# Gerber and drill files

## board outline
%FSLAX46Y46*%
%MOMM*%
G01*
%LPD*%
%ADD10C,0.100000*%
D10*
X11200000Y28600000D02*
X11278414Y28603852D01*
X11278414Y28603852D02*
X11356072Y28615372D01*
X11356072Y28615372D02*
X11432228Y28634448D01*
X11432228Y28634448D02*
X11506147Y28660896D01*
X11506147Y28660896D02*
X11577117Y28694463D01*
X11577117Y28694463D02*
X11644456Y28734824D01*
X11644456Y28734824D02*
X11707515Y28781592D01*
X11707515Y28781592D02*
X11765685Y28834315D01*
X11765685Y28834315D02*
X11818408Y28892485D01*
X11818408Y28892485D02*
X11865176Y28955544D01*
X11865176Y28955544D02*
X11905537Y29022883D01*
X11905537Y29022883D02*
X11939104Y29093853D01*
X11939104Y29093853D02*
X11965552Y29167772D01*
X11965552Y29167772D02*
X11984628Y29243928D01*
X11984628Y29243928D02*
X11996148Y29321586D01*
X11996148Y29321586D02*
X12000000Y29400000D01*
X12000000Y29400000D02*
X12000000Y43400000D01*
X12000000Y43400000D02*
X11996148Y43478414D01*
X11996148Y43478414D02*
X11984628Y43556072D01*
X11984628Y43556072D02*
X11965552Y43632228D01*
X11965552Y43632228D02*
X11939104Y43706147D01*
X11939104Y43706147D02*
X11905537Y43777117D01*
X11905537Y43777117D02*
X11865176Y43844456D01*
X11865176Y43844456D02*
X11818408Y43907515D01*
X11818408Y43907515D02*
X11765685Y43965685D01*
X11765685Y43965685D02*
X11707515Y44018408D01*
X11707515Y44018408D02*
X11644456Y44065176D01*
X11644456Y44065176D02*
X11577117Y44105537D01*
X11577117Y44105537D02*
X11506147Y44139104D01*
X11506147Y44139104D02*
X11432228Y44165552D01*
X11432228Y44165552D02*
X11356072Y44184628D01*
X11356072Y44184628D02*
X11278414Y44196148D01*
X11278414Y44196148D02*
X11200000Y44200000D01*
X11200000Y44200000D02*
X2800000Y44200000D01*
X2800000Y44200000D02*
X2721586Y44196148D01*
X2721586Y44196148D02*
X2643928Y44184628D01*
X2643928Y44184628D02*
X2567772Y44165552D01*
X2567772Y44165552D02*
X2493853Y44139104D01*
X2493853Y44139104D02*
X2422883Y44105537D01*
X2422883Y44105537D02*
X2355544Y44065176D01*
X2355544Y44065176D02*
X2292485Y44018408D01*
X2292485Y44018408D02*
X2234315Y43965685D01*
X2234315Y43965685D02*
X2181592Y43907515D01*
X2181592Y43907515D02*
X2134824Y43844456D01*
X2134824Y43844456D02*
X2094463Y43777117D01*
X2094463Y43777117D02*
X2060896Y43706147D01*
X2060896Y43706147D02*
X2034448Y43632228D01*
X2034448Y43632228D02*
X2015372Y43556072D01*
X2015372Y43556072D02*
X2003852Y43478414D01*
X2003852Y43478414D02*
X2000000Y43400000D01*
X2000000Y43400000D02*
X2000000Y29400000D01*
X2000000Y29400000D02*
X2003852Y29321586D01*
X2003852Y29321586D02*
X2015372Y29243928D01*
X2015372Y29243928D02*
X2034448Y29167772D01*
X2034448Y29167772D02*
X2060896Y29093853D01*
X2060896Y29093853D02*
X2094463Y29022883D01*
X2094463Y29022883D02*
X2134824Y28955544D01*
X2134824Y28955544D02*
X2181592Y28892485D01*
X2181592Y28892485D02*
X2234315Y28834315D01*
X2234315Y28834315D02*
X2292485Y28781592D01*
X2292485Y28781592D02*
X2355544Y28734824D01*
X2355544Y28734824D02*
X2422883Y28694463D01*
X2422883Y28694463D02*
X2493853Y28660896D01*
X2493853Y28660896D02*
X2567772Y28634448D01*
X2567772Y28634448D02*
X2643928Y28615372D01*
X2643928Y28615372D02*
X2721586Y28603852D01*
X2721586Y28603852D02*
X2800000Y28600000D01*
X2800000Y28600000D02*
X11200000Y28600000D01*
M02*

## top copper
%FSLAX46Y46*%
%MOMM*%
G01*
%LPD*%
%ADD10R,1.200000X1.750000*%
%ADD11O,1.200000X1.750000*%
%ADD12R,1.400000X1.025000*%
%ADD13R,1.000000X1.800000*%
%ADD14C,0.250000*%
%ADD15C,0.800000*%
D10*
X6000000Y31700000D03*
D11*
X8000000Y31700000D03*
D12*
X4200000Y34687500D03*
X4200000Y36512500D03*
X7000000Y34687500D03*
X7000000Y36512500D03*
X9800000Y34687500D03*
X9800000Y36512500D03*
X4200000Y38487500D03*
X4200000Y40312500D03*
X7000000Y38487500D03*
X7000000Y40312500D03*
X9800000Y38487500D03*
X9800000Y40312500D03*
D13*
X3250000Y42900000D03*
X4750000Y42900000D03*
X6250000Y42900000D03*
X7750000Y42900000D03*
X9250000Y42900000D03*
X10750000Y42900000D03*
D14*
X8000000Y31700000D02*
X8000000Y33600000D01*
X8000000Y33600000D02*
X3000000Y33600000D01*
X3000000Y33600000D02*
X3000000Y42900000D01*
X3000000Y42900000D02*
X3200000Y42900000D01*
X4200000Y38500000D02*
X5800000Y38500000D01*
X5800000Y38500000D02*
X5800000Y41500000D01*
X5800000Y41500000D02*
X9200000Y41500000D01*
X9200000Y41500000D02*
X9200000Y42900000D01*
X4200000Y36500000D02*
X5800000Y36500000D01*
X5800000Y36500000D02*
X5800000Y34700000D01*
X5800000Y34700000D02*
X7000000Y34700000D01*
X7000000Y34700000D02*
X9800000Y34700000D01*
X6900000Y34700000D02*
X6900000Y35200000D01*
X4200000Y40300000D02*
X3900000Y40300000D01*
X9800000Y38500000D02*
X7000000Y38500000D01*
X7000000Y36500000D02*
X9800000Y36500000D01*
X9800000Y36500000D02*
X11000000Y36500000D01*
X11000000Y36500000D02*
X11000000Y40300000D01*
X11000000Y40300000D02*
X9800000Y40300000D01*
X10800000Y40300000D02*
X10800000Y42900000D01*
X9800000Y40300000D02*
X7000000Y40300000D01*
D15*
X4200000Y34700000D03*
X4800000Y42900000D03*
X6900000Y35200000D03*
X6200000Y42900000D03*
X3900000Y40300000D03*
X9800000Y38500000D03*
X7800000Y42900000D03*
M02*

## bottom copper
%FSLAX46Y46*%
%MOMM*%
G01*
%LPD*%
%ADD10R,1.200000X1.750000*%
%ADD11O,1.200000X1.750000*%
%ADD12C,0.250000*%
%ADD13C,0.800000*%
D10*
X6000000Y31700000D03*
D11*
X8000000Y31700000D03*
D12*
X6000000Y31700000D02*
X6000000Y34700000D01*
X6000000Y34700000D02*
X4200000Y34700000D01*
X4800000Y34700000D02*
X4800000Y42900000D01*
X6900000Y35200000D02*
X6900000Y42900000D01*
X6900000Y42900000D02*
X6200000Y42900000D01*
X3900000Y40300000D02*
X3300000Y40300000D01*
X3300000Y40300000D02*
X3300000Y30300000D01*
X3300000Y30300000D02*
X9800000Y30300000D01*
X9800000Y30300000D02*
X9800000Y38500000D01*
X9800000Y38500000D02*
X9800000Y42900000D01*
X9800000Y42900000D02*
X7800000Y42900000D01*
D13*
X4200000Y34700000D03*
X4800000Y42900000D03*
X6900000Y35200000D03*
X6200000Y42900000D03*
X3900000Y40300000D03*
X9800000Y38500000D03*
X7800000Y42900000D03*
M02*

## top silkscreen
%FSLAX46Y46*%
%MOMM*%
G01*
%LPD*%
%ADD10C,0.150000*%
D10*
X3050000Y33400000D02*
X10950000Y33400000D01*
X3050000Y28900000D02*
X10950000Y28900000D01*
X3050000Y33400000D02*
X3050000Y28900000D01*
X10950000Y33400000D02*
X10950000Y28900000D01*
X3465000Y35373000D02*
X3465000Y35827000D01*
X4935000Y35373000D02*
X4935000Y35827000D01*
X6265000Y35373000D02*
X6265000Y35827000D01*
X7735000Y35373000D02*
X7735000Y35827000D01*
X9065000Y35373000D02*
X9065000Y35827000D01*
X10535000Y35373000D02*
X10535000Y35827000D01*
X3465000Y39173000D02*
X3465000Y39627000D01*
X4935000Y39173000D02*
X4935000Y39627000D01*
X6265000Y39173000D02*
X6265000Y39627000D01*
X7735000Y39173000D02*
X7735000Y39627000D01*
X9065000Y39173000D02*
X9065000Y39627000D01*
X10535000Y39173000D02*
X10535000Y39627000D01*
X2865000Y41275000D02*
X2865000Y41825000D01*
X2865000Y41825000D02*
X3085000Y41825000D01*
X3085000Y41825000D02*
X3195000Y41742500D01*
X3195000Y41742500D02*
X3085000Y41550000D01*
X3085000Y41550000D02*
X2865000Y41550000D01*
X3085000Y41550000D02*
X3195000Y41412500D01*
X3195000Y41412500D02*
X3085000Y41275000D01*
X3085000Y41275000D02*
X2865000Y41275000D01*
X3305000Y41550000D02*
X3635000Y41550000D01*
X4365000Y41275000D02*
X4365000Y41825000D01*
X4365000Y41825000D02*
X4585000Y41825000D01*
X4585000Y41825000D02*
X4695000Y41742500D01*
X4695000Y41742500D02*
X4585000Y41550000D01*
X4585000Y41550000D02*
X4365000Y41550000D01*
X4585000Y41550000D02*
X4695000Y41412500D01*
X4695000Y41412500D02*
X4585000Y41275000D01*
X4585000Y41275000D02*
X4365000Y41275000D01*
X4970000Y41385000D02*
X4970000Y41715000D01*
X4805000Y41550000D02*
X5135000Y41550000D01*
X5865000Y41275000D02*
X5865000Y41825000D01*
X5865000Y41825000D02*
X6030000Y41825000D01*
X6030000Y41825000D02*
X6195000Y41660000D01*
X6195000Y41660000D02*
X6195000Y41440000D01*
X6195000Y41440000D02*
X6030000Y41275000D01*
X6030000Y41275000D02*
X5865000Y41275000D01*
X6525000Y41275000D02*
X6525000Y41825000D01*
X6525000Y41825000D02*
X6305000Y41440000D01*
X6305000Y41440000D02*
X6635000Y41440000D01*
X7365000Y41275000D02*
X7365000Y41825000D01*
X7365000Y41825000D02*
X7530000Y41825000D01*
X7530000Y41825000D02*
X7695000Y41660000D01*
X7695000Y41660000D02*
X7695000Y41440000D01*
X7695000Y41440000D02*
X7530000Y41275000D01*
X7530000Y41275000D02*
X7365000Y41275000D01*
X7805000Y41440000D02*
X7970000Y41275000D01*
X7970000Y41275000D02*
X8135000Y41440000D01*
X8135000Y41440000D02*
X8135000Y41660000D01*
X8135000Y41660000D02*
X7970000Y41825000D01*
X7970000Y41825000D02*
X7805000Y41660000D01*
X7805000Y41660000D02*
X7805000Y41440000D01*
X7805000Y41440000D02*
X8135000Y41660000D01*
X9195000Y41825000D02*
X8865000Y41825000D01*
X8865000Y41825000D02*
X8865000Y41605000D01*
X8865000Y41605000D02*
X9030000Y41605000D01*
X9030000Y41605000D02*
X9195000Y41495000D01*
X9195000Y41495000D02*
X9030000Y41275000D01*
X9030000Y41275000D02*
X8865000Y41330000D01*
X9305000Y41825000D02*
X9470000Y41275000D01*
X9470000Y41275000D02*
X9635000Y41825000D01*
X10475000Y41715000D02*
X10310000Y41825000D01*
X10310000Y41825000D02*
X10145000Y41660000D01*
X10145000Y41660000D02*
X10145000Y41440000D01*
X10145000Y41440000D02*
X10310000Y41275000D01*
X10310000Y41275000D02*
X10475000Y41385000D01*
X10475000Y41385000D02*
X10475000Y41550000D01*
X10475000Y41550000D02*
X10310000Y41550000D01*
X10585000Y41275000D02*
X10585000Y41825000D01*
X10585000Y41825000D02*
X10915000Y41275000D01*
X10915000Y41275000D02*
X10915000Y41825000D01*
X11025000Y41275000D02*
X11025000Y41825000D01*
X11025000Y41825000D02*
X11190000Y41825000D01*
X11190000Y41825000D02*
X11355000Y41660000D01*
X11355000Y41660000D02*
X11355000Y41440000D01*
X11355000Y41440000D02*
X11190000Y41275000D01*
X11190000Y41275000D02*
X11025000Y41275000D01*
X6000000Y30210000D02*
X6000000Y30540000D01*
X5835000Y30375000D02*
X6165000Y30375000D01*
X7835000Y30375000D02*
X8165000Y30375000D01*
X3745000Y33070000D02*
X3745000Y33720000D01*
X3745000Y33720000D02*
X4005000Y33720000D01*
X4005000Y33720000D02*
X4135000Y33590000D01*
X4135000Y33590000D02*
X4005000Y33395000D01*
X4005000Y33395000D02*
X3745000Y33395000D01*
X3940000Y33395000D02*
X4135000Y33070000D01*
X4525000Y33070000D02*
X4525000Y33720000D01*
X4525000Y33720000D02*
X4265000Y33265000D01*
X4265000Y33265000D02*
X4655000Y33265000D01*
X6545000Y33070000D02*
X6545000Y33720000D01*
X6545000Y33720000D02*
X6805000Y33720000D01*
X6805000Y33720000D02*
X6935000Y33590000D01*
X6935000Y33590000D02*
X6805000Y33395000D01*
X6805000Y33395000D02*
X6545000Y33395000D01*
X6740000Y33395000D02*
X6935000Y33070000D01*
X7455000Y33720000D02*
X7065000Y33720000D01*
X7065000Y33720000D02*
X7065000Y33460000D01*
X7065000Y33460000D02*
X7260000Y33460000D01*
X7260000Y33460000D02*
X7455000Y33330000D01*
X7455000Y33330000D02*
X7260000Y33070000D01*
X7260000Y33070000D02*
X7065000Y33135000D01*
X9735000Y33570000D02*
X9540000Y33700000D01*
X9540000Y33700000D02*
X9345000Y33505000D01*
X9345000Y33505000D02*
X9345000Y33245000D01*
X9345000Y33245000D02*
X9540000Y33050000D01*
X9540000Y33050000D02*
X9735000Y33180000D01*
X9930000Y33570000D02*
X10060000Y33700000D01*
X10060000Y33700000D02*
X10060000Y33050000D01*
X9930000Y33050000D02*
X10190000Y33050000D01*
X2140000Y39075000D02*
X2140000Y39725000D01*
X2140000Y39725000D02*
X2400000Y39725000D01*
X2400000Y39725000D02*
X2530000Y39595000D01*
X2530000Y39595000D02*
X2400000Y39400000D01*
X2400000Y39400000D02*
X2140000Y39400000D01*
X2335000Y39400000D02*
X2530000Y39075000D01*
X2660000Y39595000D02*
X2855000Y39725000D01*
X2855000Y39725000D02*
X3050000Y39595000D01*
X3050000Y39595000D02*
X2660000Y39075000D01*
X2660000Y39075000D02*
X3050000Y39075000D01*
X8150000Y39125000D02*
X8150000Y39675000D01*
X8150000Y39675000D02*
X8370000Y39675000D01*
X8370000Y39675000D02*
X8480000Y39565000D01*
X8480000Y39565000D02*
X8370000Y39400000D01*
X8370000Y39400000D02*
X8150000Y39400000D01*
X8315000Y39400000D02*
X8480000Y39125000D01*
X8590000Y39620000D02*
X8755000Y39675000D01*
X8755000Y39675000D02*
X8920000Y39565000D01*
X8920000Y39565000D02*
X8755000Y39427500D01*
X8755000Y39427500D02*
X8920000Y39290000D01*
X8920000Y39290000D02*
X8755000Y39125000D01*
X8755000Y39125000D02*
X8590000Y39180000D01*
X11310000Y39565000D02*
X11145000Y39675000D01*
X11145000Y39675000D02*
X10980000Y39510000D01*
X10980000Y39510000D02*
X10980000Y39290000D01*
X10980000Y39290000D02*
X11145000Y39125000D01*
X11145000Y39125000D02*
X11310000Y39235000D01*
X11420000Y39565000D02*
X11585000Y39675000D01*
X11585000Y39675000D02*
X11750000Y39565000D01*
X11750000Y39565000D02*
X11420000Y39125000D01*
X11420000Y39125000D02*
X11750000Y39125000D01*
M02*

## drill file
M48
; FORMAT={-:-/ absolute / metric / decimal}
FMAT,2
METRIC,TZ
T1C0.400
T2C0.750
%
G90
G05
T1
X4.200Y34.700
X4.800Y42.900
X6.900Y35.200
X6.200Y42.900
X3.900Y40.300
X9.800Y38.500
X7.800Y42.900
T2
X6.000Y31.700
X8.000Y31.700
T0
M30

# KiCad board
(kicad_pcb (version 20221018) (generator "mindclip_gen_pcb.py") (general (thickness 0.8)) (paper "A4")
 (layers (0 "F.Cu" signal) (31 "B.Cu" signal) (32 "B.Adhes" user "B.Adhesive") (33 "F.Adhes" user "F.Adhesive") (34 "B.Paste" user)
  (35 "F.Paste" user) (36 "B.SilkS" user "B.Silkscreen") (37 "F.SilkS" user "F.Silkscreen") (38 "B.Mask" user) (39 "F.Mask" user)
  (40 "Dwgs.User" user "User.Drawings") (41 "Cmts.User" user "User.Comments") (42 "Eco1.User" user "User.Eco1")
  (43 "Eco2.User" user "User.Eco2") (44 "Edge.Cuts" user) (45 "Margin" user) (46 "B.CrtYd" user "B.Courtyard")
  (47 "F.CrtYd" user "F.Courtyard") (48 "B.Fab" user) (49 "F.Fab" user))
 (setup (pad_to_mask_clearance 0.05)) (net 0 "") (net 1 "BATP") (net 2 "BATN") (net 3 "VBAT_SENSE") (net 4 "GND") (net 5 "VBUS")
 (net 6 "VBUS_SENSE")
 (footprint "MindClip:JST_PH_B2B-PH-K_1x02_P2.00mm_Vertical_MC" (layer "F.Cu") (at 37 88.3)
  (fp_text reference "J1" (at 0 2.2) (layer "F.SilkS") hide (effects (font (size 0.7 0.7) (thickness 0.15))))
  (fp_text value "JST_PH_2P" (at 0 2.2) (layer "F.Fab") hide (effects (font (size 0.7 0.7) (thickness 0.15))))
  (fp_line (start -3.95 -1.7) (end 3.95 -1.7) (stroke (width 0.15) (type solid)) (layer "F.SilkS"))
  (fp_line (start -3.95 2.8) (end 3.95 2.8) (stroke (width 0.15) (type solid)) (layer "F.SilkS"))
  (fp_line (start -3.95 -1.7) (end -3.95 2.8) (stroke (width 0.15) (type solid)) (layer "F.SilkS"))
  (fp_line (start 3.95 -1.7) (end 3.95 2.8) (stroke (width 0.15) (type solid)) (layer "F.SilkS"))
  (pad "1" thru_hole rect (at -1 0) (size 1.2 1.75) (drill 0.75) (layers "*.Cu" "*.Mask") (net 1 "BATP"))
  (pad "2" thru_hole oval (at 1 0) (size 1.2 1.75) (drill 0.75) (layers "*.Cu" "*.Mask") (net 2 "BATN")))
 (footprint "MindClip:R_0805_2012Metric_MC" (layer "F.Cu") (at 34.2 84.4 90)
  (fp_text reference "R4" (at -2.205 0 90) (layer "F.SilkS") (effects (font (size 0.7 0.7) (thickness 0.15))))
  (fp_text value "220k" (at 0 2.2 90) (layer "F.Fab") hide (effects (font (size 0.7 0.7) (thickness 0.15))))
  (fp_line (start -0.227 -0.735) (end 0.227 -0.735) (stroke (width 0.15) (type solid)) (layer "F.SilkS"))
  (fp_line (start -0.227 0.735) (end 0.227 0.735) (stroke (width 0.15) (type solid)) (layer "F.SilkS"))
  (pad "1" smd rect (at -0.9125 0 90) (size 1.025 1.4) (layers "F.Cu" "F.Paste" "F.Mask") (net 1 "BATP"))
  (pad "2" smd rect (at 0.9125 0 90) (size 1.025 1.4) (layers "F.Cu" "F.Paste" "F.Mask") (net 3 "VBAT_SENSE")))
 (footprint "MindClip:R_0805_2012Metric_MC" (layer "F.Cu") (at 37 84.4 90)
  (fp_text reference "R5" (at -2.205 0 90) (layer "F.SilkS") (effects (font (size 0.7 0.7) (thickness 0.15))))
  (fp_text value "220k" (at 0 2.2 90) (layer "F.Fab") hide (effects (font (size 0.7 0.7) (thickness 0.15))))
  (fp_line (start -0.227 -0.735) (end 0.227 -0.735) (stroke (width 0.15) (type solid)) (layer "F.SilkS"))
  (fp_line (start -0.227 0.735) (end 0.227 0.735) (stroke (width 0.15) (type solid)) (layer "F.SilkS"))
  (pad "1" smd rect (at -0.9125 0 90) (size 1.025 1.4) (layers "F.Cu" "F.Paste" "F.Mask") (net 3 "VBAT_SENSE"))
  (pad "2" smd rect (at 0.9125 0 90) (size 1.025 1.4) (layers "F.Cu" "F.Paste" "F.Mask") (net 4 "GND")))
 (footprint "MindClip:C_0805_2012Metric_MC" (layer "F.Cu") (at 39.8 84.4 90)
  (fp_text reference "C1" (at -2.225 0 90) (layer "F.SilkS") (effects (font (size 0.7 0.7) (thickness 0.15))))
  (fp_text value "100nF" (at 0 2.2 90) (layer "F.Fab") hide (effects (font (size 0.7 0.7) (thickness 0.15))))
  (fp_line (start -0.227 -0.735) (end 0.227 -0.735) (stroke (width 0.15) (type solid)) (layer "F.SilkS"))
  (fp_line (start -0.227 0.735) (end 0.227 0.735) (stroke (width 0.15) (type solid)) (layer "F.SilkS"))
  (pad "1" smd rect (at -0.9125 0 90) (size 1.025 1.4) (layers "F.Cu" "F.Paste" "F.Mask") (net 3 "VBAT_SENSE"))
  (pad "2" smd rect (at 0.9125 0 90) (size 1.025 1.4) (layers "F.Cu" "F.Paste" "F.Mask") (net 4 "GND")))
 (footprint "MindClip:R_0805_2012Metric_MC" (layer "F.Cu") (at 34.2 80.6 90)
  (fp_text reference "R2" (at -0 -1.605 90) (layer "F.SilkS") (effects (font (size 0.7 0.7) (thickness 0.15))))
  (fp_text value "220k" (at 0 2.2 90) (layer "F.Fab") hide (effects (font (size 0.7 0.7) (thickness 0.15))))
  (fp_line (start -0.227 -0.735) (end 0.227 -0.735) (stroke (width 0.15) (type solid)) (layer "F.SilkS"))
  (fp_line (start -0.227 0.735) (end 0.227 0.735) (stroke (width 0.15) (type solid)) (layer "F.SilkS"))
  (pad "1" smd rect (at -0.9125 0 90) (size 1.025 1.4) (layers "F.Cu" "F.Paste" "F.Mask") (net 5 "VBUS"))
  (pad "2" smd rect (at 0.9125 0 90) (size 1.025 1.4) (layers "F.Cu" "F.Paste" "F.Mask") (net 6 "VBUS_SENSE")))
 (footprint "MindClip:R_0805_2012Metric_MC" (layer "F.Cu") (at 37 80.6 90)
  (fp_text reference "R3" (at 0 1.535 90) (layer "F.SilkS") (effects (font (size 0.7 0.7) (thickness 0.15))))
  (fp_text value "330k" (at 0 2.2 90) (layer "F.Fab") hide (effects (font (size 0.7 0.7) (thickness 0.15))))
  (fp_line (start -0.227 -0.735) (end 0.227 -0.735) (stroke (width 0.15) (type solid)) (layer "F.SilkS"))
  (fp_line (start -0.227 0.735) (end 0.227 0.735) (stroke (width 0.15) (type solid)) (layer "F.SilkS"))
  (pad "1" smd rect (at -0.9125 0 90) (size 1.025 1.4) (layers "F.Cu" "F.Paste" "F.Mask") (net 6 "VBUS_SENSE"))
  (pad "2" smd rect (at 0.9125 0 90) (size 1.025 1.4) (layers "F.Cu" "F.Paste" "F.Mask") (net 4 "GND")))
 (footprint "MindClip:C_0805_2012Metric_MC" (layer "F.Cu") (at 39.8 80.6 90)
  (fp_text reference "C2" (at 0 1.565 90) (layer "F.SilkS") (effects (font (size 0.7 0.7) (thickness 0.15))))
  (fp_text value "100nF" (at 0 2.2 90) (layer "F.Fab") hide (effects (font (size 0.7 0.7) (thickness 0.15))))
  (fp_line (start -0.227 -0.735) (end 0.227 -0.735) (stroke (width 0.15) (type solid)) (layer "F.SilkS"))
  (fp_line (start -0.227 0.735) (end 0.227 0.735) (stroke (width 0.15) (type solid)) (layer "F.SilkS"))
  (pad "1" smd rect (at -0.9125 0 90) (size 1.025 1.4) (layers "F.Cu" "F.Paste" "F.Mask") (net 6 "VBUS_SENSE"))
  (pad "2" smd rect (at 0.9125 0 90) (size 1.025 1.4) (layers "F.Cu" "F.Paste" "F.Mask") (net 4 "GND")))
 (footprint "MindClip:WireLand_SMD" (layer "F.Cu") (at 37 77.1)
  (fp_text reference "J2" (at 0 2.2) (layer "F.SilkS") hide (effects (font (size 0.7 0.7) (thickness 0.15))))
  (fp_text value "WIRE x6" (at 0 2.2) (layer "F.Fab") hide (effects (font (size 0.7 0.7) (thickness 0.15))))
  (pad "1" smd rect (at -3.75 0) (size 1 1.8) (layers "F.Cu" "F.Paste" "F.Mask") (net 2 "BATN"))
  (pad "2" smd rect (at -2.25 0) (size 1 1.8) (layers "F.Cu" "F.Paste" "F.Mask") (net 1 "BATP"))
  (pad "3" smd rect (at -0.75 0) (size 1 1.8) (layers "F.Cu" "F.Paste" "F.Mask") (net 3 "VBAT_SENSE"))
  (pad "4" smd rect (at 0.75 0) (size 1 1.8) (layers "F.Cu" "F.Paste" "F.Mask") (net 6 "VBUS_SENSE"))
  (pad "5" smd rect (at 2.25 0) (size 1 1.8) (layers "F.Cu" "F.Paste" "F.Mask") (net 5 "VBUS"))
  (pad "6" smd rect (at 3.75 0) (size 1 1.8) (layers "F.Cu" "F.Paste" "F.Mask") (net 4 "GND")))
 (gr_line (start 32.8 91.4) (end 41.2 91.4) (stroke (width 0.1) (type solid)) (layer "Edge.Cuts"))
 (gr_line (start 42 90.6) (end 42 76.6) (stroke (width 0.1) (type solid)) (layer "Edge.Cuts"))
 (gr_line (start 41.2 75.8) (end 32.8 75.8) (stroke (width 0.1) (type solid)) (layer "Edge.Cuts"))
 (gr_line (start 32 76.6) (end 32 90.6) (stroke (width 0.1) (type solid)) (layer "Edge.Cuts"))
 (gr_arc (start 41.2 91.4) (mid 41.7657 91.1657) (end 42 90.6) (stroke (width 0.1) (type solid)) (layer "Edge.Cuts"))
 (gr_arc (start 42 76.6) (mid 41.7657 76.0343) (end 41.2 75.8) (stroke (width 0.1) (type solid)) (layer "Edge.Cuts"))
 (gr_arc (start 32.8 75.8) (mid 32.2343 76.0343) (end 32 76.6) (stroke (width 0.1) (type solid)) (layer "Edge.Cuts"))
 (gr_arc (start 32 90.6) (mid 32.2343 91.1657) (end 32.8 91.4) (stroke (width 0.1) (type solid)) (layer "Edge.Cuts"))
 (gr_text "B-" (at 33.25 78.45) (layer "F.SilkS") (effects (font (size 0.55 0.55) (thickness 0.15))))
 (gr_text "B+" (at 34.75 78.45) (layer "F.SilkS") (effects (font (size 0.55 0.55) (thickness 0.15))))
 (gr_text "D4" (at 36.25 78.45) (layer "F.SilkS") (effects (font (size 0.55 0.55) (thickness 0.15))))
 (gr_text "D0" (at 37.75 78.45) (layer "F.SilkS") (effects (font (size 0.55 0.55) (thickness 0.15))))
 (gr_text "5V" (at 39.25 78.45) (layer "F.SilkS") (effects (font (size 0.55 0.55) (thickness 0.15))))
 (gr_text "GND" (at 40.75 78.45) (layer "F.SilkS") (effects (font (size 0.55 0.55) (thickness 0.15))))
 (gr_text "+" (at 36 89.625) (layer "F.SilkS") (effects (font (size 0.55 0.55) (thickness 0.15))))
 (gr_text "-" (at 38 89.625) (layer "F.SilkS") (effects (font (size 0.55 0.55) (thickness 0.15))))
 (segment (start 38 88.3) (end 38 86.4) (width 0.25) (layer "F.Cu") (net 2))
 (segment (start 38 86.4) (end 33 86.4) (width 0.25) (layer "F.Cu") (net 2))
 (segment (start 33 86.4) (end 33 77.1) (width 0.25) (layer "F.Cu") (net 2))
 (segment (start 33 77.1) (end 33.2 77.1) (width 0.25) (layer "F.Cu") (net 2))
 (segment (start 34.2 81.5) (end 35.8 81.5) (width 0.25) (layer "F.Cu") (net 5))
 (segment (start 35.8 81.5) (end 35.8 78.5) (width 0.25) (layer "F.Cu") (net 5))
 (segment (start 35.8 78.5) (end 39.2 78.5) (width 0.25) (layer "F.Cu") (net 5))
 (segment (start 39.2 78.5) (end 39.2 77.1) (width 0.25) (layer "F.Cu") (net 5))
 (segment (start 36 88.3) (end 36 85.3) (width 0.25) (layer "B.Cu") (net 1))
 (segment (start 36 85.3) (end 34.2 85.3) (width 0.25) (layer "B.Cu") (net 1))
 (segment (start 34.8 85.3) (end 34.8 77.1) (width 0.25) (layer "B.Cu") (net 1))
 (segment (start 34.2 83.5) (end 35.8 83.5) (width 0.25) (layer "F.Cu") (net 3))
 (segment (start 35.8 83.5) (end 35.8 85.3) (width 0.25) (layer "F.Cu") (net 3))
 (segment (start 35.8 85.3) (end 37 85.3) (width 0.25) (layer "F.Cu") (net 3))
 (segment (start 37 85.3) (end 39.8 85.3) (width 0.25) (layer "F.Cu") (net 3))
 (segment (start 36.9 85.3) (end 36.9 84.8) (width 0.25) (layer "F.Cu") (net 3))
 (segment (start 36.9 84.8) (end 36.9 77.1) (width 0.25) (layer "B.Cu") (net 3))
 (segment (start 36.9 77.1) (end 36.2 77.1) (width 0.25) (layer "B.Cu") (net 3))
 (segment (start 34.2 79.7) (end 33.9 79.7) (width 0.25) (layer "F.Cu") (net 6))
 (segment (start 33.9 79.7) (end 33.3 79.7) (width 0.25) (layer "B.Cu") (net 6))
 (segment (start 33.3 79.7) (end 33.3 89.7) (width 0.25) (layer "B.Cu") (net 6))
 (segment (start 33.3 89.7) (end 39.8 89.7) (width 0.25) (layer "B.Cu") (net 6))
 (segment (start 39.8 89.7) (end 39.8 81.5) (width 0.25) (layer "B.Cu") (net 6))
 (segment (start 39.8 81.5) (end 37 81.5) (width 0.25) (layer "F.Cu") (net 6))
 (segment (start 39.8 81.5) (end 39.8 77.1) (width 0.25) (layer "B.Cu") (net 6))
 (segment (start 39.8 77.1) (end 37.8 77.1) (width 0.25) (layer "B.Cu") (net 6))
 (segment (start 37 83.5) (end 39.8 83.5) (width 0.25) (layer "F.Cu") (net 4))
 (segment (start 39.8 83.5) (end 41 83.5) (width 0.25) (layer "F.Cu") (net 4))
 (segment (start 41 83.5) (end 41 79.7) (width 0.25) (layer "F.Cu") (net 4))
 (segment (start 41 79.7) (end 39.8 79.7) (width 0.25) (layer "F.Cu") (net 4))
 (segment (start 40.8 79.7) (end 40.8 77.1) (width 0.25) (layer "F.Cu") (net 4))
 (segment (start 39.8 79.7) (end 37 79.7) (width 0.25) (layer "F.Cu") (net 4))
 (via (at 34.2 85.3) (size 0.8) (drill 0.4) (layers "F.Cu" "B.Cu") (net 1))
 (via (at 34.8 77.1) (size 0.8) (drill 0.4) (layers "F.Cu" "B.Cu") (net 1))
 (via (at 36.9 84.8) (size 0.8) (drill 0.4) (layers "F.Cu" "B.Cu") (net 3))
 (via (at 36.2 77.1) (size 0.8) (drill 0.4) (layers "F.Cu" "B.Cu") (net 3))
 (via (at 33.9 79.7) (size 0.8) (drill 0.4) (layers "F.Cu" "B.Cu") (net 6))
 (via (at 39.8 81.5) (size 0.8) (drill 0.4) (layers "F.Cu" "B.Cu") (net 6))
 (via (at 37.8 77.1) (size 0.8) (drill 0.4) (layers "F.Cu" "B.Cu") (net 6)))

